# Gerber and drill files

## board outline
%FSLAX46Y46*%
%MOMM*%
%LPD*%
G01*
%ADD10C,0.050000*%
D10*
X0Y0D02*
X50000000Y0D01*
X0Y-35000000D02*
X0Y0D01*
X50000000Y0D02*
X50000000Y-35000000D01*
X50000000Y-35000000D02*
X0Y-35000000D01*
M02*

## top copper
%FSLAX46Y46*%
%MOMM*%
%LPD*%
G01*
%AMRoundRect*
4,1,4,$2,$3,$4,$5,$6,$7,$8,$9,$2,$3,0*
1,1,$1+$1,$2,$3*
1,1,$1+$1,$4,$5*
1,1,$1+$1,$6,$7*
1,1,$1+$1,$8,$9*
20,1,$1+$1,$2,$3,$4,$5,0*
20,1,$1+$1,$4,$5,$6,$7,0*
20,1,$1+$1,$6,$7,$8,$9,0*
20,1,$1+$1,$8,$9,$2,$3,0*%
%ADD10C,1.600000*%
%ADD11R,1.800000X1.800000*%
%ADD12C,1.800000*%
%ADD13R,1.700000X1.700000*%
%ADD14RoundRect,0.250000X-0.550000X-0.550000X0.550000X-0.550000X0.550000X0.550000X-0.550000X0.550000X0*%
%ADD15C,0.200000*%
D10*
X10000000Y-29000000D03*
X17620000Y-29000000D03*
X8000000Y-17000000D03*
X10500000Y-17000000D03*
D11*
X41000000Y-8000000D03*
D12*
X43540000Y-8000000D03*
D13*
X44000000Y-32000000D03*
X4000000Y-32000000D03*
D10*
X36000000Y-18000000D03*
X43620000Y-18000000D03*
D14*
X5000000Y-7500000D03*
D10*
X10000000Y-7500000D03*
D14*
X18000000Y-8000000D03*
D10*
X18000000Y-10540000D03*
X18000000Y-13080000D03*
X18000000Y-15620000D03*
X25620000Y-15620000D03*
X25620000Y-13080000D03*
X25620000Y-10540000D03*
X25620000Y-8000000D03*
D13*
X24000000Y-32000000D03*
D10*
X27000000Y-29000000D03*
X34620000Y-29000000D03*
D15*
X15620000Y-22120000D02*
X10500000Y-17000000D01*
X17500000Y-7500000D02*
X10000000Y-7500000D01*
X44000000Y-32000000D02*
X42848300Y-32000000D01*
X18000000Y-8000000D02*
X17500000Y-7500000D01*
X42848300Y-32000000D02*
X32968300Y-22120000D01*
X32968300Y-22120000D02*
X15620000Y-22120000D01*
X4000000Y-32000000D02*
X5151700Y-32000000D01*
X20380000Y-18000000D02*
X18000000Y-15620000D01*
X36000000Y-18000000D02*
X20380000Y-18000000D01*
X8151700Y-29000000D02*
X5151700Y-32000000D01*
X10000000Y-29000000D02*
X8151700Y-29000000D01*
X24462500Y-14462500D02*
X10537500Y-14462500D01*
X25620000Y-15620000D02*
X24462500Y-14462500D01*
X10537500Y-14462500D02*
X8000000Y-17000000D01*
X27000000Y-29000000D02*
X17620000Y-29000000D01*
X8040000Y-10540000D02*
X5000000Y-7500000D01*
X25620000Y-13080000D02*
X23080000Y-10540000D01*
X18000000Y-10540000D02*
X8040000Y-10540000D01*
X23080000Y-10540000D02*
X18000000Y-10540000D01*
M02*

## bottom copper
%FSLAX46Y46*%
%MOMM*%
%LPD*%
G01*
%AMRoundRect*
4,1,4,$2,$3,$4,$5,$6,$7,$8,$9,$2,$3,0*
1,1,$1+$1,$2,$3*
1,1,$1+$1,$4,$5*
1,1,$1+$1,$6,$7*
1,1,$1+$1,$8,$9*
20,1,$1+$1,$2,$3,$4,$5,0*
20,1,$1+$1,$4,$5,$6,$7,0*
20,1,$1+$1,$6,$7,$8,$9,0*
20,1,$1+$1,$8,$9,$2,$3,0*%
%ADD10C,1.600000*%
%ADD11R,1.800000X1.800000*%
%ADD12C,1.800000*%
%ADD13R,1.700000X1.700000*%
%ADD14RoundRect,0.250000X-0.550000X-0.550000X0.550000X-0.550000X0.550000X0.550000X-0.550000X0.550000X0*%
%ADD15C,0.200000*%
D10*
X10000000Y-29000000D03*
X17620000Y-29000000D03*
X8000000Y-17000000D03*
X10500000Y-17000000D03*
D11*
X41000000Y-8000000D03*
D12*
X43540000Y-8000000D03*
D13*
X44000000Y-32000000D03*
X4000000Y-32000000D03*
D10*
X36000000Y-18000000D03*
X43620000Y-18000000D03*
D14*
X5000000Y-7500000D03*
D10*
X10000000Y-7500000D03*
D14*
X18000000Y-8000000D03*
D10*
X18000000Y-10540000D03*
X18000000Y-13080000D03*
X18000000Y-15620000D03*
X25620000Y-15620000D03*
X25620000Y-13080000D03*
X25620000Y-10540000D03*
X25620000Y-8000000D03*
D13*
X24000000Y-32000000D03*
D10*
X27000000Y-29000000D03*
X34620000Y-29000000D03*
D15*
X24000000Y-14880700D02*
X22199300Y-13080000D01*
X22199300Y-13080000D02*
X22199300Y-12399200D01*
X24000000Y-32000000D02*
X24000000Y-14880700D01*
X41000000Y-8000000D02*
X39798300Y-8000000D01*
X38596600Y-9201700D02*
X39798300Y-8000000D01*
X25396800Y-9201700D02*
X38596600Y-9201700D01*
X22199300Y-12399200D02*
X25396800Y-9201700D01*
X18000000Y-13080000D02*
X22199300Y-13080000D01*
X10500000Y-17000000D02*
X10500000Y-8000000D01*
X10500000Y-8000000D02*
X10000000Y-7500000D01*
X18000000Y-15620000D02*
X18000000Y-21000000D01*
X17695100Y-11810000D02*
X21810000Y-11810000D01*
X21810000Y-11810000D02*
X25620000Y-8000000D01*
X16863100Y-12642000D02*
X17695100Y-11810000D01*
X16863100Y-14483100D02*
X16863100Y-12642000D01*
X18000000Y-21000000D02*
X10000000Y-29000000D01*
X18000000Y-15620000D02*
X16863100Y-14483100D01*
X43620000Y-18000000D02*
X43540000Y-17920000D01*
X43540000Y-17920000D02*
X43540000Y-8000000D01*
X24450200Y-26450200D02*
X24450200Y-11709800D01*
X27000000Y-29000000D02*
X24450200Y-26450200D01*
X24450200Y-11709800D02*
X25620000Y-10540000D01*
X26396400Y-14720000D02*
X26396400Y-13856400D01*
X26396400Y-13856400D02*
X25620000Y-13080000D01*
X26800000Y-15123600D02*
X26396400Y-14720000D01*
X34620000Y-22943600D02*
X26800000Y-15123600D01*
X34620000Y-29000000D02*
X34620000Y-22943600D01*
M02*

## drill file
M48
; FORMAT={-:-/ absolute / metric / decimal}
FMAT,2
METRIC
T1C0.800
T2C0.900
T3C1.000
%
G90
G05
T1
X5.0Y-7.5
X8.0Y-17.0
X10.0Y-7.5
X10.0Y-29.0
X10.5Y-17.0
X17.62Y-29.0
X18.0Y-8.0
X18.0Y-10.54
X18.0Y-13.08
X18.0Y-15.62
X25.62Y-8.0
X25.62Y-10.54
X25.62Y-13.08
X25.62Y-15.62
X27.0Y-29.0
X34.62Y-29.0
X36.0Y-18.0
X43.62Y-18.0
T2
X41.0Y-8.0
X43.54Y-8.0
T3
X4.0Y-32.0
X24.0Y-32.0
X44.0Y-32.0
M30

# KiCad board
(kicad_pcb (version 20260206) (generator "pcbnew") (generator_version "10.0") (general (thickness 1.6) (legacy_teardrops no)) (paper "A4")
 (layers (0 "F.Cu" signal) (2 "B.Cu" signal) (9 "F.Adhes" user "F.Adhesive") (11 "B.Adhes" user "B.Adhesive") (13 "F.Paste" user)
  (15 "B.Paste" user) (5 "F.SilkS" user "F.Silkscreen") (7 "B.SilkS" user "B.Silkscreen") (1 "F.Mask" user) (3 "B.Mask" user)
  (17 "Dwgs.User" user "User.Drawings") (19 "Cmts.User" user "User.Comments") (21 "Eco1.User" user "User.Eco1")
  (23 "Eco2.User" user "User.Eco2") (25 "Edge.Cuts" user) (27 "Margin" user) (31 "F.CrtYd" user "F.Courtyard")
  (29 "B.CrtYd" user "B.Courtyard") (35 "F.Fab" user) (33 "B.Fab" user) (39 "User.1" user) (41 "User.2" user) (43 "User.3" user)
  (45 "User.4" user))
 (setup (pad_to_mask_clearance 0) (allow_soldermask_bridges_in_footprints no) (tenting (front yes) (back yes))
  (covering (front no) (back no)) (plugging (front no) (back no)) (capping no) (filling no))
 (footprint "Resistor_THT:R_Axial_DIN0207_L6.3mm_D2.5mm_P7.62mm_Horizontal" (layer "F.Cu") (at 10 29)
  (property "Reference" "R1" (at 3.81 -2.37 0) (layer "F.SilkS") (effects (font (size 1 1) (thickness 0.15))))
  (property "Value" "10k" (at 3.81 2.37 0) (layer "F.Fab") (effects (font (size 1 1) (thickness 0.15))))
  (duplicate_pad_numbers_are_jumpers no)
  (pad "1" thru_hole circle (at 0 0) (size 1.6 1.6) (drill 0.8) (layers "*.Cu" "*.Mask") (remove_unused_layers no) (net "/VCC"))
  (pad "2" thru_hole circle (at 7.62 0) (size 1.6 1.6) (drill 0.8) (layers "*.Cu" "*.Mask") (remove_unused_layers no) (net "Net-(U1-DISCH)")))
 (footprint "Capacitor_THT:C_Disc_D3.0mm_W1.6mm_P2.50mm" (layer "F.Cu") (at 8 17)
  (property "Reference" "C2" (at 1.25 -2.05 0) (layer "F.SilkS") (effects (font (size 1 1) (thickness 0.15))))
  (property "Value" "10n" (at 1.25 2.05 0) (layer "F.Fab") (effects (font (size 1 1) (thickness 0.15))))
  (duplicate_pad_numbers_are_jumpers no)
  (pad "1" thru_hole circle (at 0 0) (size 1.6 1.6) (drill 0.8) (layers "*.Cu" "*.Mask") (remove_unused_layers no) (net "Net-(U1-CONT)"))
  (pad "2" thru_hole circle (at 2.5 0) (size 1.6 1.6) (drill 0.8) (layers "*.Cu" "*.Mask") (remove_unused_layers no) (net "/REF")))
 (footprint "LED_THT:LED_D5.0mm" (layer "F.Cu") (at 41 8)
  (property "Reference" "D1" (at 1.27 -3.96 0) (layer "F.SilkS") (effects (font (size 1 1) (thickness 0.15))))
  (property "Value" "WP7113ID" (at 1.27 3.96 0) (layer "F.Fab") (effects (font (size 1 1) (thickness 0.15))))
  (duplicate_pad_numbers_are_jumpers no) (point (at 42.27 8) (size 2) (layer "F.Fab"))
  (pad "1" thru_hole rect (at 0 0) (size 1.8 1.8) (drill 0.9) (layers "*.Cu" "*.Mask") (remove_unused_layers no) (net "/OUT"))
  (pad "2" thru_hole circle (at 2.54 0) (size 1.8 1.8) (drill 0.9) (layers "*.Cu" "*.Mask") (remove_unused_layers no) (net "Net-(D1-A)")))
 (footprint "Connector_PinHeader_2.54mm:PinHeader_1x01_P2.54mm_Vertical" (layer "F.Cu") (at 44 32)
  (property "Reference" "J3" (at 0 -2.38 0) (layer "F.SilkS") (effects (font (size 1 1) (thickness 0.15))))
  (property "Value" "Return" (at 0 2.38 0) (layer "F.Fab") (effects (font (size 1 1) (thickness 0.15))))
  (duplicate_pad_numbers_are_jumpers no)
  (pad "1" thru_hole rect (at 0 0) (size 1.7 1.7) (drill 1) (layers "*.Cu" "*.Mask") (remove_unused_layers no) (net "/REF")))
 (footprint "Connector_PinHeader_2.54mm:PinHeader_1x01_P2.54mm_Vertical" (layer "F.Cu") (at 4 32)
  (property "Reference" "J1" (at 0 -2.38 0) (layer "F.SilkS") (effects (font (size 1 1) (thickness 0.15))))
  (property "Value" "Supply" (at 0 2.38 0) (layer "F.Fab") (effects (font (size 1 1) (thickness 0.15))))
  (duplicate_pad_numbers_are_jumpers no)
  (pad "1" thru_hole rect (at 0 0) (size 1.7 1.7) (drill 1) (layers "*.Cu" "*.Mask") (remove_unused_layers no) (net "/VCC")))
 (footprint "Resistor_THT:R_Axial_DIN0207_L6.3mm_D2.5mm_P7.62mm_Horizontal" (layer "F.Cu") (at 36 18)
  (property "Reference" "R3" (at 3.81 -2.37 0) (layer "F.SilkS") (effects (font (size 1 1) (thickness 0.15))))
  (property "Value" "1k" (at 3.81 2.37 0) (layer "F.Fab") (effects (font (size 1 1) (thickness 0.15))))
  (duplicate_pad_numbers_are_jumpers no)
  (pad "1" thru_hole circle (at 0 0) (size 1.6 1.6) (drill 0.8) (layers "*.Cu" "*.Mask") (remove_unused_layers no) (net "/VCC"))
  (pad "2" thru_hole circle (at 7.62 0) (size 1.6 1.6) (drill 0.8) (layers "*.Cu" "*.Mask") (remove_unused_layers no) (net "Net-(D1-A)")))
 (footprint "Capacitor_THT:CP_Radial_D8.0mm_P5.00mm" (layer "F.Cu") (at 5 7.5)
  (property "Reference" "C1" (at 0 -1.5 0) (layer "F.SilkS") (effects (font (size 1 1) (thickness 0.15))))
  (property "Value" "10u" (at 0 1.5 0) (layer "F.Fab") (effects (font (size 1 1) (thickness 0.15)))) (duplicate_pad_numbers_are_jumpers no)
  (pad "1" thru_hole roundrect (at 0 0) (size 1.6 1.6) (drill 0.8) (layers "*.Cu" "*.Mask") (remove_unused_layers no)
   (roundrect_rratio 0.15625) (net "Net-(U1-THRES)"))
  (pad "2" thru_hole circle (at 5 0) (size 1.6 1.6) (drill 0.8) (layers "*.Cu" "*.Mask") (remove_unused_layers no) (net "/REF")))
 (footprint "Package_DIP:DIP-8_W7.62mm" (layer "F.Cu") (at 18 8)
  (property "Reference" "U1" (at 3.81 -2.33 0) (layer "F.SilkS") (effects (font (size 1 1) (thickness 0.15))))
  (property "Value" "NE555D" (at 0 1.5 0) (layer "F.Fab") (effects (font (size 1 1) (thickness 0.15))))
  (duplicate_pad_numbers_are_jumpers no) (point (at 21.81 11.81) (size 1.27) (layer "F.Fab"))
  (pad "1" thru_hole roundrect (at 0 0) (size 1.6 1.6) (drill 0.8) (layers "*.Cu" "*.Mask") (remove_unused_layers no)
   (roundrect_rratio 0.15625) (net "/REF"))
  (pad "2" thru_hole circle (at 0 2.54) (size 1.6 1.6) (drill 0.8) (layers "*.Cu" "*.Mask") (remove_unused_layers no) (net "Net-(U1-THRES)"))
  (pad "3" thru_hole circle (at 0 5.08) (size 1.6 1.6) (drill 0.8) (layers "*.Cu" "*.Mask") (remove_unused_layers no) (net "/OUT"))
  (pad "4" thru_hole circle (at 0 7.62) (size 1.6 1.6) (drill 0.8) (layers "*.Cu" "*.Mask") (remove_unused_layers no) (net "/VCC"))
  (pad "5" thru_hole circle (at 7.62 7.62) (size 1.6 1.6) (drill 0.8) (layers "*.Cu" "*.Mask") (remove_unused_layers no)
   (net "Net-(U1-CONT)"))
  (pad "6" thru_hole circle (at 7.62 5.08) (size 1.6 1.6) (drill 0.8) (layers "*.Cu" "*.Mask") (remove_unused_layers no)
   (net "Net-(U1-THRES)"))
  (pad "7" thru_hole circle (at 7.62 2.54) (size 1.6 1.6) (drill 0.8) (layers "*.Cu" "*.Mask") (remove_unused_layers no)
   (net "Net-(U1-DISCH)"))
  (pad "8" thru_hole circle (at 7.62 0) (size 1.6 1.6) (drill 0.8) (layers "*.Cu" "*.Mask") (remove_unused_layers no) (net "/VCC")))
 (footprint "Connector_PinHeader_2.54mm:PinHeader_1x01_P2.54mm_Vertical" (layer "F.Cu") (at 24 32)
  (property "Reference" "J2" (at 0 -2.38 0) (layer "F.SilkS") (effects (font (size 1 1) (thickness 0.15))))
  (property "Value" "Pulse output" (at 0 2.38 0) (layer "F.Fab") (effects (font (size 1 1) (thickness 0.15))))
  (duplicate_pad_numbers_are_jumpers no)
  (pad "1" thru_hole rect (at 0 0) (size 1.7 1.7) (drill 1) (layers "*.Cu" "*.Mask") (remove_unused_layers no) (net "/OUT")))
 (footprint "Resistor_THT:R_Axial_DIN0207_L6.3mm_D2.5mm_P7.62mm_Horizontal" (layer "F.Cu") (at 27 29)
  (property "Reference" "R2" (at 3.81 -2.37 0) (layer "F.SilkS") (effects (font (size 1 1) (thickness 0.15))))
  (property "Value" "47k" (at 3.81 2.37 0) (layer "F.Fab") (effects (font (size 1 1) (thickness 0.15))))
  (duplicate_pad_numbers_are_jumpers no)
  (pad "1" thru_hole circle (at 0 0) (size 1.6 1.6) (drill 0.8) (layers "*.Cu" "*.Mask") (remove_unused_layers no) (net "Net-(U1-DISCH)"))
  (pad "2" thru_hole circle (at 7.62 0) (size 1.6 1.6) (drill 0.8) (layers "*.Cu" "*.Mask") (remove_unused_layers no) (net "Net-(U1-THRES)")))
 (gr_line (start 0 0) (end 50 0) (stroke (width 0.05) (type default)) (layer "Edge.Cuts"))
 (gr_line (start 0 35) (end 0 0) (stroke (width 0.05) (type default)) (layer "Edge.Cuts"))
 (gr_line (start 50 0) (end 50 35) (stroke (width 0.05) (type default)) (layer "Edge.Cuts"))
 (gr_line (start 50 35) (end 0 35) (stroke (width 0.05) (type default)) (layer "Edge.Cuts"))
 (segment (start 24 14.8807) (end 22.1993 13.08) (width 0.200000) (layer "B.Cu") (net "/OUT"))
 (segment (start 22.1993 13.08) (end 22.1993 12.3992) (width 0.2) (layer "B.Cu") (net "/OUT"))
 (segment (start 24 32) (end 24 14.8807) (width 0.2) (layer "B.Cu") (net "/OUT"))
 (segment (start 41 8) (end 39.7983 8) (width 0.2) (layer "B.Cu") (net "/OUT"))
 (segment (start 38.5966 9.2017) (end 39.7983 8) (width 0.2) (layer "B.Cu") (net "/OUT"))
 (segment (start 25.3968 9.2017) (end 38.5966 9.2017) (width 0.2) (layer "B.Cu") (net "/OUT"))
 (segment (start 22.1993 12.3992) (end 25.3968 9.2017) (width 0.2) (layer "B.Cu") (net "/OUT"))
 (segment (start 18 13.08) (end 22.1993 13.08) (width 0.2) (layer "B.Cu") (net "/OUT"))
 (segment (start 15.62 22.12) (end 10.5 17) (width 0.2) (layer "F.Cu") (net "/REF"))
 (segment (start 17.5 7.5) (end 10 7.5) (width 0.2) (layer "F.Cu") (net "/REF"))
 (segment (start 44 32) (end 42.8483 32) (width 0.2) (layer "F.Cu") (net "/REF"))
 (segment (start 18 8) (end 17.5 7.5) (width 0.2) (layer "F.Cu") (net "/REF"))
 (segment (start 42.8483 32) (end 32.9683 22.12) (width 0.2) (layer "F.Cu") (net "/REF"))
 (segment (start 32.9683 22.12) (end 15.62 22.12) (width 0.2) (layer "F.Cu") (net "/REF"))
 (segment (start 10.5 17) (end 10.5 8) (width 0.2) (layer "B.Cu") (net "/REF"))
 (segment (start 10.5 8) (end 10 7.5) (width 0.2) (layer "B.Cu") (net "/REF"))
 (segment (start 4 32) (end 5.1517 32) (width 0.2) (layer "F.Cu") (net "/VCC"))
 (segment (start 20.38 18) (end 18 15.62) (width 0.2) (layer "F.Cu") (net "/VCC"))
 (segment (start 36 18) (end 20.38 18) (width 0.2) (layer "F.Cu") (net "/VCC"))
 (segment (start 8.1517 29) (end 5.1517 32) (width 0.2) (layer "F.Cu") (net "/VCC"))
 (segment (start 10 29) (end 8.1517 29) (width 0.2) (layer "F.Cu") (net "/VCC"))
 (segment (start 18 15.62) (end 18 21) (width 0.2) (layer "B.Cu") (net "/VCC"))
 (segment (start 17.6951 11.81) (end 21.81 11.81) (width 0.2) (layer "B.Cu") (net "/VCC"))
 (segment (start 21.81 11.81) (end 25.62 8) (width 0.2) (layer "B.Cu") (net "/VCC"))
 (segment (start 16.8631 12.642) (end 17.6951 11.81) (width 0.2) (layer "B.Cu") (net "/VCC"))
 (segment (start 16.8631 14.4831) (end 16.8631 12.642) (width 0.2) (layer "B.Cu") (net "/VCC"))
 (segment (start 18 21) (end 10 29) (width 0.2) (layer "B.Cu") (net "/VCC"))
 (segment (start 18 15.62) (end 16.8631 14.4831) (width 0.2) (layer "B.Cu") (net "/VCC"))
 (segment (start 43.62 18) (end 43.54 17.92) (width 0.2) (layer "B.Cu") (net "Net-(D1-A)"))
 (segment (start 43.54 17.92) (end 43.54 8) (width 0.2) (layer "B.Cu") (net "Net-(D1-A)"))
 (segment (start 24.4625 14.4625) (end 10.5375 14.4625) (width 0.2) (layer "F.Cu") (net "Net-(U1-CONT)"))
 (segment (start 25.62 15.62) (end 24.4625 14.4625) (width 0.2) (layer "F.Cu") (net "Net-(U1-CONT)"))
 (segment (start 10.5375 14.4625) (end 8 17) (width 0.2) (layer "F.Cu") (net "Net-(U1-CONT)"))
 (segment (start 27 29) (end 17.62 29) (width 0.2) (layer "F.Cu") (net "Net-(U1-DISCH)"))
 (segment (start 24.4502 26.4502) (end 24.4502 11.7098) (width 0.2) (layer "B.Cu") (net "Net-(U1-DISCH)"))
 (segment (start 27 29) (end 24.4502 26.4502) (width 0.2) (layer "B.Cu") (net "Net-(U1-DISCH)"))
 (segment (start 24.4502 11.7098) (end 25.62 10.54) (width 0.2) (layer "B.Cu") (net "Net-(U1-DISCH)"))
 (segment (start 8.04 10.54) (end 5 7.5) (width 0.2) (layer "F.Cu") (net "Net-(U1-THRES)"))
 (segment (start 25.62 13.08) (end 23.08 10.54) (width 0.2) (layer "F.Cu") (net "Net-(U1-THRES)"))
 (segment (start 18 10.54) (end 8.04 10.54) (width 0.2) (layer "F.Cu") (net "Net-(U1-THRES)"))
 (segment (start 23.08 10.54) (end 18 10.54) (width 0.2) (layer "F.Cu") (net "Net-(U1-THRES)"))
 (segment (start 26.3964 14.72) (end 26.3964 13.8564) (width 0.2) (layer "B.Cu") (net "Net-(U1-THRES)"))
 (segment (start 26.3964 13.8564) (end 25.62 13.08) (width 0.2) (layer "B.Cu") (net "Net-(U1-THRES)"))
 (segment (start 26.8 15.1236) (end 26.3964 14.72) (width 0.2) (layer "B.Cu") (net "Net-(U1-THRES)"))
 (segment (start 34.62 22.9436) (end 26.8 15.1236) (width 0.2) (layer "B.Cu") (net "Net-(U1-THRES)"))
 (segment (start 34.62 29) (end 34.62 22.9436) (width 0.2) (layer "B.Cu") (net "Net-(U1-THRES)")))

